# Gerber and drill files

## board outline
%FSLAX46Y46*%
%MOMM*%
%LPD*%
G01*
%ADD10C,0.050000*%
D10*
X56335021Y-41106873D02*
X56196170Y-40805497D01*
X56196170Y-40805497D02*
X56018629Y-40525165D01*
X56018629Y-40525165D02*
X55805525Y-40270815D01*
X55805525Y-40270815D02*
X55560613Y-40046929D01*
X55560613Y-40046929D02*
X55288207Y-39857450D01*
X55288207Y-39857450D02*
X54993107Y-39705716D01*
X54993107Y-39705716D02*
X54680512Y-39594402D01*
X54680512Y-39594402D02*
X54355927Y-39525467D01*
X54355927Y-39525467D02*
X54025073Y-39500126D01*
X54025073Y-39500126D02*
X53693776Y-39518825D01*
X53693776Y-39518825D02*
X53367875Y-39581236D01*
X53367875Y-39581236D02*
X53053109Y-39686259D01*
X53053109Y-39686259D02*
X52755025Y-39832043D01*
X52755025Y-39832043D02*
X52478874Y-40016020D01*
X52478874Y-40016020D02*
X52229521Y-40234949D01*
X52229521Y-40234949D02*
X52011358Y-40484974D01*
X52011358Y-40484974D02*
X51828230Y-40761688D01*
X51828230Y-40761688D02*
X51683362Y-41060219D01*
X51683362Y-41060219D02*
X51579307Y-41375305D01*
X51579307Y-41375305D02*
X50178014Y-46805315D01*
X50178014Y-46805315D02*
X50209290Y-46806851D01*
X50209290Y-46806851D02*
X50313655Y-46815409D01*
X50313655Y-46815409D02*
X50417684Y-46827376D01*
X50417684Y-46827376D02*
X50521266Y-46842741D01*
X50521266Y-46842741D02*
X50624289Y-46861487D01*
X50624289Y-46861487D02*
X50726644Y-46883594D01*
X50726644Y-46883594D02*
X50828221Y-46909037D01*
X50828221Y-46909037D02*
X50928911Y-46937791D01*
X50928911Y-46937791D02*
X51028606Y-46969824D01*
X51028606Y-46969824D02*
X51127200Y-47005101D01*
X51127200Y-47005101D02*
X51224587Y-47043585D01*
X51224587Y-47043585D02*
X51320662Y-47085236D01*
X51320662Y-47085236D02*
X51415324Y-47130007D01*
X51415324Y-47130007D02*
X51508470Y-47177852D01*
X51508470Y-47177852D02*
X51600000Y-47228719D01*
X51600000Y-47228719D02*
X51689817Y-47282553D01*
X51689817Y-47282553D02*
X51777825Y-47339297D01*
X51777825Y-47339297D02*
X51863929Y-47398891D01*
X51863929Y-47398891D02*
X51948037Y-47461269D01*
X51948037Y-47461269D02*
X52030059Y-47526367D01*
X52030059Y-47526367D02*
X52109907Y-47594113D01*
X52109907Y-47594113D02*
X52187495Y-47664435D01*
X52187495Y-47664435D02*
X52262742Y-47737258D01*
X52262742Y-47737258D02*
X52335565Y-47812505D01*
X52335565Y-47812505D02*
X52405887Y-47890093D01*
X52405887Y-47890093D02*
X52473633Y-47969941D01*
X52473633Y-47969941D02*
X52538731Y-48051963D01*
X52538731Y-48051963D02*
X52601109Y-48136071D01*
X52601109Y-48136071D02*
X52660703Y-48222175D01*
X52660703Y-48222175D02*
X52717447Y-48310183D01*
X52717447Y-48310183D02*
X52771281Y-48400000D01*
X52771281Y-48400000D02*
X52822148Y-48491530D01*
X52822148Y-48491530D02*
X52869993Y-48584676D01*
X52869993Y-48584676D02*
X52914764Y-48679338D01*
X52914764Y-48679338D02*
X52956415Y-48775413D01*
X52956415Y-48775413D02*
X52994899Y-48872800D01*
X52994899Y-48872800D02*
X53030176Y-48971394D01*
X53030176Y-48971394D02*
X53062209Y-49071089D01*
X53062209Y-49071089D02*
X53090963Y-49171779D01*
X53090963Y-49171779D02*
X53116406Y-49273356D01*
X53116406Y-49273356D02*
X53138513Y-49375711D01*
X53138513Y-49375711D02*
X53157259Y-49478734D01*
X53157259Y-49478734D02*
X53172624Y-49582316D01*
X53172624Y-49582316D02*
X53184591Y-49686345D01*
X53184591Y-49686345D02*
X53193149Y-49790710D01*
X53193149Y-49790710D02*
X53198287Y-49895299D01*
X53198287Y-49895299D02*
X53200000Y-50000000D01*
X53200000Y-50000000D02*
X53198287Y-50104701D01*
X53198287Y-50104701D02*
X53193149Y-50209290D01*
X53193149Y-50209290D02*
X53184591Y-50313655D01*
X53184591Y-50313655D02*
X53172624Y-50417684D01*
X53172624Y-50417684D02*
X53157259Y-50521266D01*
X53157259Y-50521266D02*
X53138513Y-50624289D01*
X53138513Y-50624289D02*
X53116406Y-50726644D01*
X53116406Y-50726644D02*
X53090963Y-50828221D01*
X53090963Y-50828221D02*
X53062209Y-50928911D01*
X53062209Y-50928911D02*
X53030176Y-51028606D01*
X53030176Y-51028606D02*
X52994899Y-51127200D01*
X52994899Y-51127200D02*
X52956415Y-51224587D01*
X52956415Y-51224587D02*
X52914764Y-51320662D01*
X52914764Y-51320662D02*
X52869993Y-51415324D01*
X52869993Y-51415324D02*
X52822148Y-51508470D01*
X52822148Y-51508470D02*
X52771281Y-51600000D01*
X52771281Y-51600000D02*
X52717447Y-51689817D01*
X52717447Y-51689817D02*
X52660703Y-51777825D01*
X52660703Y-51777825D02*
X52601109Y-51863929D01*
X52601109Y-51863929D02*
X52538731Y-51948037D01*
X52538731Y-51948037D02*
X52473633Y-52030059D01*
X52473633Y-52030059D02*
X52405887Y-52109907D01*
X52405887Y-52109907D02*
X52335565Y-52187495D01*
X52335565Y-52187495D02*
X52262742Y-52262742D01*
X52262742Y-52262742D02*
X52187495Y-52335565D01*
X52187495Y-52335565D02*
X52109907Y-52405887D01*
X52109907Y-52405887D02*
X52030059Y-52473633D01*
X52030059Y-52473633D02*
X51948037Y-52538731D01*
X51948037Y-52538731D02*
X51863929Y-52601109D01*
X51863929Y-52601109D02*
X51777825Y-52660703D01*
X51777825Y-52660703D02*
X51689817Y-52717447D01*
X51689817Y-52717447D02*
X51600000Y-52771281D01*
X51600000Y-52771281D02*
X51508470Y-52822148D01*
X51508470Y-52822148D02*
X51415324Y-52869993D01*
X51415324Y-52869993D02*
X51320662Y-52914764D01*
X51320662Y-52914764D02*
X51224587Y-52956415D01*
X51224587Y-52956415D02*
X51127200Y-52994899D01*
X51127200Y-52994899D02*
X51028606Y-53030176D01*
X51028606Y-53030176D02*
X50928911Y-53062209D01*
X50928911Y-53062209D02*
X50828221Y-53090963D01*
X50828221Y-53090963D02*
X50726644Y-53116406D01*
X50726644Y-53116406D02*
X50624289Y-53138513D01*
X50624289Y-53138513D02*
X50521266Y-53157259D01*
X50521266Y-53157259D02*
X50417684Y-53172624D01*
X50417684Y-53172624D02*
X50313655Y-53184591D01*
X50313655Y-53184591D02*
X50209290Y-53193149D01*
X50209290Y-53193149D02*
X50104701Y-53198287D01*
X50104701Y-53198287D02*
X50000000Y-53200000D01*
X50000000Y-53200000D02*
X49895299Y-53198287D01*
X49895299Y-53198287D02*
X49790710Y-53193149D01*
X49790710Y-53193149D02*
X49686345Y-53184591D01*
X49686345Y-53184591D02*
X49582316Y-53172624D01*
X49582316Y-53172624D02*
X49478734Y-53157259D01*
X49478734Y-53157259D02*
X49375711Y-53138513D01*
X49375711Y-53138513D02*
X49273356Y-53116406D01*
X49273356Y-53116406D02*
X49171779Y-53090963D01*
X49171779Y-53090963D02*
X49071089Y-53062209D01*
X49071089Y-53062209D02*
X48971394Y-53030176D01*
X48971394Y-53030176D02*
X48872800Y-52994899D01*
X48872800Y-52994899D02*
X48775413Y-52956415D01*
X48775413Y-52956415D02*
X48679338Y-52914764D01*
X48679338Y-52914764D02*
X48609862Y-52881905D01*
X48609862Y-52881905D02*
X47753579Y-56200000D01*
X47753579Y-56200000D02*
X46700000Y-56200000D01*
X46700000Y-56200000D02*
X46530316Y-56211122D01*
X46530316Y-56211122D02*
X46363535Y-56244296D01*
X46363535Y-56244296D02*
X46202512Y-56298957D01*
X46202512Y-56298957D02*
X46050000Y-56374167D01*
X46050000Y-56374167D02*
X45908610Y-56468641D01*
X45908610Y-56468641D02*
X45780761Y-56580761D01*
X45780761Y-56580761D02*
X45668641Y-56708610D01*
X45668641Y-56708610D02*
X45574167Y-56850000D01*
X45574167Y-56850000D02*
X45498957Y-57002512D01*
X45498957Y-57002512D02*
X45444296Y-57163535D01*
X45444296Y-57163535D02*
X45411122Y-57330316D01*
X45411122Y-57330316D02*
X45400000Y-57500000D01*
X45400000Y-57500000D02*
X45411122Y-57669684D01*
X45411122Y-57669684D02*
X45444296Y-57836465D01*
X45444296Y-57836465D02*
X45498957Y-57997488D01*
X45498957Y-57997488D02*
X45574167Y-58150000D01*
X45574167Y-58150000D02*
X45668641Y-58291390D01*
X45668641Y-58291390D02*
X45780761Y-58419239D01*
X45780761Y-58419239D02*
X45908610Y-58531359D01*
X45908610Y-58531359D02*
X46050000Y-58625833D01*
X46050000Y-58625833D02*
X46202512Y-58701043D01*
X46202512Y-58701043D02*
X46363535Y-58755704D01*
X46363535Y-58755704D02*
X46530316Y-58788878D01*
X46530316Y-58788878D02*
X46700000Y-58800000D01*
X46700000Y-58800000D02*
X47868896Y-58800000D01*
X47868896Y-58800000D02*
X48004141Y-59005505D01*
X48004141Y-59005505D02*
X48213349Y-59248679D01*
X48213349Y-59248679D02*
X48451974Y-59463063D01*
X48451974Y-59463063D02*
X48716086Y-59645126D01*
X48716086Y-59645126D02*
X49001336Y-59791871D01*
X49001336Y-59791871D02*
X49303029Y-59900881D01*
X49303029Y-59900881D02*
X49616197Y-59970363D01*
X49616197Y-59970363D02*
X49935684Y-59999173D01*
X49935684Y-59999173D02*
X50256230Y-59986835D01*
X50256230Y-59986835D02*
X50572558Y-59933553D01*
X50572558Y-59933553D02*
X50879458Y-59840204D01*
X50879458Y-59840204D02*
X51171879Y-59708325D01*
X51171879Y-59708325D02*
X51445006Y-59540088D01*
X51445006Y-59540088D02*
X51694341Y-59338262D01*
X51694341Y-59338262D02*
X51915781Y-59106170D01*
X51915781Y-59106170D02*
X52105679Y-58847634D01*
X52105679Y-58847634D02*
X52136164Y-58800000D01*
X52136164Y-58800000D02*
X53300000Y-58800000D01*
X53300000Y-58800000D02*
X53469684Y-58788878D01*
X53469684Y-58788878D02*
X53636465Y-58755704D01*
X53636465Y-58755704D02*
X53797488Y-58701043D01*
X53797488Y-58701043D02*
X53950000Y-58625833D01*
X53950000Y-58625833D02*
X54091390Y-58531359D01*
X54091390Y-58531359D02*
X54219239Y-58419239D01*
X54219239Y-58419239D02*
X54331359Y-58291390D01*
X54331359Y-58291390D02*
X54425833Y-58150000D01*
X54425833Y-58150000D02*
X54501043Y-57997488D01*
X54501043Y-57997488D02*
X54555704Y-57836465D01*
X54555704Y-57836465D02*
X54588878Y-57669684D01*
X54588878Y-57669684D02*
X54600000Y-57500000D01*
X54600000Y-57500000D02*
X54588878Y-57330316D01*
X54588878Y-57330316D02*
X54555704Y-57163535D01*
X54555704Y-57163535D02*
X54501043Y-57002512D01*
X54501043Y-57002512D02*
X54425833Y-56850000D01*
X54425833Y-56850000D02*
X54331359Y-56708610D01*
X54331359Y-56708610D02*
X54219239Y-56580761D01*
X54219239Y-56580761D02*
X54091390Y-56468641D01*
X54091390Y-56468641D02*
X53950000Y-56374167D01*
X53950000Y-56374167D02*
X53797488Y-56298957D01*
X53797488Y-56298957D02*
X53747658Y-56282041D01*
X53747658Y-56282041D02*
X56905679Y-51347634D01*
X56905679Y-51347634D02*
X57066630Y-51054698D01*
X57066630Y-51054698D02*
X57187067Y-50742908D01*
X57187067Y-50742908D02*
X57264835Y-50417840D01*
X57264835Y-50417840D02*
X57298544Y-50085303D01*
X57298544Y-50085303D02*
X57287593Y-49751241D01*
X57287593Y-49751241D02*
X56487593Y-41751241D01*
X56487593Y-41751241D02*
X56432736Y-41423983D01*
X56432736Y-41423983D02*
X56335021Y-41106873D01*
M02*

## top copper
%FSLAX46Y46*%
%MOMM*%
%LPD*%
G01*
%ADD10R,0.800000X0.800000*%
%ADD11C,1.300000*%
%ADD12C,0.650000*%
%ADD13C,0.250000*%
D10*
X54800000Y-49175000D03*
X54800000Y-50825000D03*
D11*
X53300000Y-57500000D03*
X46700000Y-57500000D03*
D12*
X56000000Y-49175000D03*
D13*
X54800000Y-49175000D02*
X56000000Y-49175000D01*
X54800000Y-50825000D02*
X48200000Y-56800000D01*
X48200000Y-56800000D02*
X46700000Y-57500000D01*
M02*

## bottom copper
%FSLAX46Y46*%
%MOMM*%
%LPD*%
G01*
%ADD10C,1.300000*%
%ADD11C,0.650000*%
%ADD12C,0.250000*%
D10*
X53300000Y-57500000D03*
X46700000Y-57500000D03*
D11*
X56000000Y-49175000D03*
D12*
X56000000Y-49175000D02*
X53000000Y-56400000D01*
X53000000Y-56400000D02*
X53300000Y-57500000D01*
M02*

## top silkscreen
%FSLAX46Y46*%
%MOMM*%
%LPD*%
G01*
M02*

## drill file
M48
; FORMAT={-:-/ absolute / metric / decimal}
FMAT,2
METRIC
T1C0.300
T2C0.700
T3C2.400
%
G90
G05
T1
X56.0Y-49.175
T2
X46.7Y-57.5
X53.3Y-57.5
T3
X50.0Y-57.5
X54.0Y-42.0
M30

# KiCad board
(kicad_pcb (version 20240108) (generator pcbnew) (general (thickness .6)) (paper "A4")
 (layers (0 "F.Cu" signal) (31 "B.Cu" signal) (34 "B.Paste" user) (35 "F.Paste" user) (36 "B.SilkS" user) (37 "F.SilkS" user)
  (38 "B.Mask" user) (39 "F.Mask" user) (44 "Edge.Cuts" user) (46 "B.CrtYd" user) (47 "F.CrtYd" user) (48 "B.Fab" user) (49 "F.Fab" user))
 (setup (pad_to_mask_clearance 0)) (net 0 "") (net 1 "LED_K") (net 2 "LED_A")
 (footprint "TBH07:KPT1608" (layer "F.Cu") (at 54.8 50)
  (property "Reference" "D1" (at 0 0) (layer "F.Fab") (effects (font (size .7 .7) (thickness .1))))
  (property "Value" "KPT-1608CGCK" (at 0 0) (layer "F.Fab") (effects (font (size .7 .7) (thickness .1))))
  (pad "1" smd rect (at 0 -.825) (size .8 .8) (layers "F.Cu" "F.Paste" "F.Mask") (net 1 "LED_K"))
  (pad "2" smd rect (at 0 .825) (size .8 .8) (layers "F.Cu" "F.Paste" "F.Mask") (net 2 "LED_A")))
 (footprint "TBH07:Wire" (layer "F.Cu") (at 53.3 57.5)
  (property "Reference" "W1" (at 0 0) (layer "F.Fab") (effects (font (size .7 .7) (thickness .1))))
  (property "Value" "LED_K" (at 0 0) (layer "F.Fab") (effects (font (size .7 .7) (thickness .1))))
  (pad "1" thru_hole circle (at 0 0) (size 1.3 1.3) (drill .7) (layers "*.Cu" "*.Mask") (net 1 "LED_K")))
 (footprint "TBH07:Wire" (layer "F.Cu") (at 46.7 57.5)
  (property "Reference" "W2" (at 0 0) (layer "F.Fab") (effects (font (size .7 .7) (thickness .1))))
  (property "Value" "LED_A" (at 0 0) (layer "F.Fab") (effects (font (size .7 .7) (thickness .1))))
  (pad "1" thru_hole circle (at 0 0) (size 1.3 1.3) (drill .7) (layers "*.Cu" "*.Mask") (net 2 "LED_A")))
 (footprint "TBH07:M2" (layer "F.Cu") (at 54 42)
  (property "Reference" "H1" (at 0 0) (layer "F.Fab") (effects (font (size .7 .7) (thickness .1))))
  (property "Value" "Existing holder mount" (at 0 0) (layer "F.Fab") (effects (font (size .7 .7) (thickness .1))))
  (pad "" np_thru_hole circle (at 0 0) (size 2.4 2.4) (drill 2.4) (layers "*.Cu" "*.Mask")))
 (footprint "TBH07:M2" (layer "F.Cu") (at 50 57.5)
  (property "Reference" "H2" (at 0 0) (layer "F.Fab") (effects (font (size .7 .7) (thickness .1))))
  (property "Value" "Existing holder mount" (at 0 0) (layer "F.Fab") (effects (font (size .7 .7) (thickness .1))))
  (pad "" np_thru_hole circle (at 0 0) (size 2.4 2.4) (drill 2.4) (layers "*.Cu" "*.Mask")))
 (segment (start 54.8 49.175) (end 56 49.175) (width .25) (layer "F.Cu") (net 1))
 (via (at 56 49.175) (size .65) (drill .3) (layers "F.Cu" "B.Cu") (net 1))
 (segment (start 56 49.175) (end 53.0 56.4) (width .25) (layer "B.Cu") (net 1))
 (segment (start 53.0 56.4) (end 53.3 57.5) (width .25) (layer "B.Cu") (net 1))
 (segment (start 54.8 50.825) (end 48.2 56.8) (width .25) (layer "F.Cu") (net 2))
 (segment (start 48.2 56.8) (end 46.7 57.5) (width .25) (layer "F.Cu") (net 2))
 (gr_line (start 56.33502112309573 41.106872710809505) (end 56.19616994221303 40.80549692971512) (stroke (width .05) (type default))
  (layer "Edge.Cuts"))
 (gr_line (start 56.19616994221303 40.80549692971512) (end 56.018628567749545 40.525164854817525) (stroke (width .05) (type default))
  (layer "Edge.Cuts"))
 (gr_line (start 56.018628567749545 40.525164854817525) (end 55.80552476774115 40.27081513045213) (stroke (width .05) (type default))
  (layer "Edge.Cuts"))
 (gr_line (start 55.80552476774115 40.27081513045213) (end 55.56061281780951 40.04692866671782) (stroke (width .05) (type default))
  (layer "Edge.Cuts"))
 (gr_line (start 55.56061281780951 40.04692866671782) (end 55.28820736163088 39.857449698737504) (stroke (width .05) (type default))
  (layer "Edge.Cuts"))
 (gr_line (start 55.28820736163088 39.857449698737504) (end 54.99310739933244 39.70571630058723) (stroke (width .05) (type default))
  (layer "Edge.Cuts"))
 (gr_line (start 54.99310739933244 39.70571630058723) (end 54.68051174292211 39.594401578038195) (stroke (width .05) (type default))
  (layer "Edge.Cuts"))
 (gr_line (start 54.68051174292211 39.594401578038195) (end 54.35592742818367 39.52546657612661) (stroke (width .05) (type default))
  (layer "Edge.Cuts"))
 (gr_line (start 54.35592742818367 39.52546657612661) (end 54.02507269655606 39.500125731184184) (stroke (width .05) (type default))
  (layer "Edge.Cuts"))
 (gr_line (start 54.02507269655606 39.500125731184184) (end 53.69377625617691 39.51882547596527) (stroke (width .05) (type default))
  (layer "Edge.Cuts"))
 (gr_line (start 53.69377625617691 39.51882547596527) (end 53.36787459682077 39.5812363747866) (stroke (width .05) (type default))
  (layer "Edge.Cuts"))
 (gr_line (start 53.36787459682077 39.5812363747866) (end 53.05310916774729 39.686258927235855) (stroke (width .05) (type default))
  (layer "Edge.Cuts"))
 (gr_line (start 53.05310916774729 39.686258927235855) (end 52.75502522988974 39.83204293820452) (stroke (width .05) (type default))
  (layer "Edge.Cuts"))
 (gr_line (start 52.75502522988974 39.83204293820452) (end 52.47887416431721 40.01602011300055) (stroke (width .05) (type default))
  (layer "Edge.Cuts"))
 (gr_line (start 52.47887416431721 40.01602011300055) (end 52.22952095801417 40.23494930330912) (stroke (width .05) (type default))
  (layer "Edge.Cuts"))
 (gr_line (start 52.22952095801417 40.23494930330912) (end 52.011358496811724 40.484973606897526) (stroke (width .05) (type default))
  (layer "Edge.Cuts"))
 (gr_line (start 52.011358496811724 40.484973606897526) (end 51.82823017538246 40.76168831513197) (stroke (width .05) (type default))
  (layer "Edge.Cuts"))
 (gr_line (start 51.82823017538246 40.76168831513197) (end 51.683362187687976 41.0602185112665) (stroke (width .05) (type default))
  (layer "Edge.Cuts"))
 (gr_line (start 51.683362187687976 41.0602185112665) (end 51.579306690726604 41.375304952445575) (stroke (width .05) (type default))
  (layer "Edge.Cuts"))
 (gr_line (start 51.579306690726604 41.375304952445575) (end 50.17801378986232 46.805314943294675) (stroke (width .05) (type default))
  (layer "Edge.Cuts"))
 (gr_line (start 50.17801378986232 46.805314943294675) (end 50.20929001353646 46.80685144563647) (stroke (width .05) (type default))
  (layer "Edge.Cuts"))
 (gr_line (start 50.20929001353646 46.80685144563647) (end 50.31365484905459 46.815408874648966) (stroke (width .05) (type default))
  (layer "Edge.Cuts"))
 (gr_line (start 50.31365484905459 46.815408874648966) (end 50.41768381510416 46.827376443603804) (stroke (width .05) (type default))
  (layer "Edge.Cuts"))
 (gr_line (start 50.41768381510416 46.827376443603804) (end 50.521265514862684 46.842741337328384) (stroke (width .05) (type default))
  (layer "Edge.Cuts"))
 (gr_line (start 50.521265514862684 46.842741337328384) (end 50.624289030451614 46.86148710270966) (stroke (width .05) (type default))
  (layer "Edge.Cuts"))
 (gr_line (start 50.624289030451614 46.86148710270966) (end 50.726644041709996 46.883593666312535) (stroke (width .05) (type default))
  (layer "Edge.Cuts"))
 (gr_line (start 50.726644041709996 46.883593666312535) (end 50.828220944328066 46.90903735587498) (stroke (width .05) (type default))
  (layer "Edge.Cuts"))
 (gr_line (start 50.828220944328066 46.90903735587498) (end 50.92891096721428 46.937790925656934) (stroke (width .05) (type default))
  (layer "Edge.Cuts"))
 (gr_line (start 50.92891096721428 46.937790925656934) (end 51.02860628897012 46.969823585615664) (stroke (width .05) (type default))
  (layer "Edge.Cuts"))
 (gr_line (start 51.02860628897012 46.969823585615664) (end 51.12720015334795 47.00510103437656) (stroke (width .05) (type default))
  (layer "Edge.Cuts"))
 (gr_line (start 51.12720015334795 47.00510103437656) (end 51.22458698356829 47.04358549596388) (stroke (width .05) (type default))
  (layer "Edge.Cuts"))
 (gr_line (start 51.22458698356829 47.04358549596388) (end 51.320662495374066 47.08523576025224) (stroke (width .05) (type default))
  (layer "Edge.Cuts"))
 (gr_line (start 51.320662495374066 47.08523576025224) (end 51.415323808700805 47.1300072270954) (stroke (width .05) (type default))
  (layer "Edge.Cuts"))
 (gr_line (start 51.415323808700805 47.1300072270954) (end 51.50846955784319 47.17785195408526) (stroke (width .05) (type default))
  (layer "Edge.Cuts"))
 (gr_line (start 51.50846955784319 47.17785195408526) (end 51.6 47.2287187078898) (stroke (width .05) (type default)) (layer "Edge.Cuts"))
 (gr_line (start 51.6 47.2287187078898) (end 51.68981712208118 47.28255301911495) (stroke (width .05) (type default)) (layer "Edge.Cuts"))
 (gr_line (start 51.68981712208118 47.28255301911495) (end 51.77782474566273 47.33929724063186) (stroke (width .05) (type default))
  (layer "Edge.Cuts"))
 (gr_line (start 51.77782474566273 47.33929724063186) (end 51.86392862997697 47.39889060930683) (stroke (width .05) (type default))
  (layer "Edge.Cuts"))
 (gr_line (start 51.86392862997697 47.39889060930683) (end 51.9480365728279 47.46126931106805) (stroke (width .05) (type default))
  (layer "Edge.Cuts"))
 (gr_line (start 51.9480365728279 47.46126931106805) (end 52.030058509323666 47.52636654923924) (stroke (width .05) (type default))
  (layer "Edge.Cuts"))
 (gr_line (start 52.030058509323666 47.52636654923924) (end 52.10990660832022 47.59411261606727) (stroke (width .05) (type default))
  (layer "Edge.Cuts"))
 (gr_line (start 52.10990660832022 47.59411261606727) (end 52.187495366473186 47.66443496736693) (stroke (width .05) (type default))
  (layer "Edge.Cuts"))
 (gr_line (start 52.187495366473186 47.66443496736693) (end 52.262741699796955 47.737258300203045) (stroke (width .05) (type default))
  (layer "Edge.Cuts"))
 (gr_line (start 52.262741699796955 47.737258300203045) (end 52.33556503263308 47.812504633526814) (stroke (width .05) (type default))
  (layer "Edge.Cuts"))
 (gr_line (start 52.33556503263308 47.812504633526814) (end 52.40588738393273 47.89009339167978) (stroke (width .05) (type default))
  (layer "Edge.Cuts"))
 (gr_line (start 52.40588738393273 47.89009339167978) (end 52.47363345076076 47.969941490676334) (stroke (width .05) (type default))
  (layer "Edge.Cuts"))
 (gr_line (start 52.47363345076076 47.969941490676334) (end 52.538730688931956 48.0519634271721) (stroke (width .05) (type default))
  (layer "Edge.Cuts"))
 (gr_line (start 52.538730688931956 48.0519634271721) (end 52.60110939069317 48.13607137002303) (stroke (width .05) (type default))
  (layer "Edge.Cuts"))
 (gr_line (start 52.60110939069317 48.13607137002303) (end 52.66070275936814 48.22217525433727) (stroke (width .05) (type default))
  (layer "Edge.Cuts"))
 (gr_line (start 52.66070275936814 48.22217525433727) (end 52.71744698088505 48.31018287791882) (stroke (width .05) (type default))
  (layer "Edge.Cuts"))
 (gr_line (start 52.71744698088505 48.31018287791882) (end 52.7712812921102 48.4) (stroke (width .05) (type default)) (layer "Edge.Cuts"))
 (gr_line (start 52.7712812921102 48.4) (end 52.82214804591474 48.49153044215681) (stroke (width .05) (type default)) (layer "Edge.Cuts"))
 (gr_line (start 52.82214804591474 48.49153044215681) (end 52.8699927729046 48.584676191299195) (stroke (width .05) (type default))
  (layer "Edge.Cuts"))
 (gr_line (start 52.8699927729046 48.584676191299195) (end 52.91476423974776 48.679337504625934) (stroke (width .05) (type default))
  (layer "Edge.Cuts"))
 (gr_line (start 52.91476423974776 48.679337504625934) (end 52.95641450403612 48.77541301643171) (stroke (width .05) (type default))
  (layer "Edge.Cuts"))
 (gr_line (start 52.95641450403612 48.77541301643171) (end 52.99489896562344 48.87279984665205) (stroke (width .05) (type default))
  (layer "Edge.Cuts"))
 (gr_line (start 52.99489896562344 48.87279984665205) (end 53.030176414384336 48.97139371102988) (stroke (width .05) (type default))
  (layer "Edge.Cuts"))
 (gr_line (start 53.030176414384336 48.97139371102988) (end 53.062209074343066 49.07108903278572) (stroke (width .05) (type default))
  (layer "Edge.Cuts"))
 (gr_line (start 53.062209074343066 49.07108903278572) (end 53.09096264412502 49.171779055671934) (stroke (width .05) (type default))
  (layer "Edge.Cuts"))
 (gr_line (start 53.09096264412502 49.171779055671934) (end 53.116406333687465 49.273355958290004) (stroke (width .05) (type default))
  (layer "Edge.Cuts"))
 (gr_line (start 53.116406333687465 49.273355958290004) (end 53.13851289729034 49.375710969548386) (stroke (width .05) (type default))
  (layer "Edge.Cuts"))
 (gr_line (start 53.13851289729034 49.375710969548386) (end 53.157258662671616 49.478734485137316) (stroke (width .05) (type default))
  (layer "Edge.Cuts"))
 (gr_line (start 53.157258662671616 49.478734485137316) (end 53.172623556396196 49.58231618489584) (stroke (width .05) (type default))
  (layer "Edge.Cuts"))
 (gr_line (start 53.172623556396196 49.58231618489584) (end 53.184591125351034 49.68634515094541) (stroke (width .05) (type default))
  (layer "Edge.Cuts"))
 (gr_line (start 53.184591125351034 49.68634515094541) (end 53.19314855436353 49.79070998646354) (stroke (width .05) (type default))
  (layer "Edge.Cuts"))
 (gr_line (start 53.19314855436353 49.79070998646354) (end 53.19828667992437 49.89529893497031) (stroke (width .05) (type default))
  (layer "Edge.Cuts"))
 (gr_line (start 53.19828667992437 49.89529893497031) (end 53.2 50.0) (stroke (width .05) (type default)) (layer "Edge.Cuts"))
 (gr_line (start 53.2 50.0) (end 53.19828667992437 50.10470106502969) (stroke (width .05) (type default)) (layer "Edge.Cuts"))
 (gr_line (start 53.19828667992437 50.10470106502969) (end 53.19314855436353 50.20929001353646) (stroke (width .05) (type default))
  (layer "Edge.Cuts"))
 (gr_line (start 53.19314855436353 50.20929001353646) (end 53.184591125351034 50.31365484905459) (stroke (width .05) (type default))
  (layer "Edge.Cuts"))
 (gr_line (start 53.184591125351034 50.31365484905459) (end 53.17262355639619 50.41768381510417) (stroke (width .05) (type default))
  (layer "Edge.Cuts"))
 (gr_line (start 53.17262355639619 50.41768381510417) (end 53.157258662671616 50.521265514862684) (stroke (width .05) (type default))
  (layer "Edge.Cuts"))
 (gr_line (start 53.157258662671616 50.521265514862684) (end 53.13851289729034 50.624289030451614) (stroke (width .05) (type default))
  (layer "Edge.Cuts"))
 (gr_line (start 53.13851289729034 50.624289030451614) (end 53.116406333687465 50.726644041709996) (stroke (width .05) (type default))
  (layer "Edge.Cuts"))
 (gr_line (start 53.116406333687465 50.726644041709996) (end 53.09096264412502 50.828220944328066) (stroke (width .05) (type default))
  (layer "Edge.Cuts"))
 (gr_line (start 53.09096264412502 50.828220944328066) (end 53.062209074343066 50.928910967214286) (stroke (width .05) (type default))
  (layer "Edge.Cuts"))
 (gr_line (start 53.062209074343066 50.928910967214286) (end 53.030176414384336 51.02860628897012) (stroke (width .05) (type default))
  (layer "Edge.Cuts"))
 (gr_line (start 53.030176414384336 51.02860628897012) (end 52.99489896562344 51.12720015334795) (stroke (width .05) (type default))
  (layer "Edge.Cuts"))
 (gr_line (start 52.99489896562344 51.12720015334795) (end 52.95641450403612 51.22458698356829) (stroke (width .05) (type default))
  (layer "Edge.Cuts"))
 (gr_line (start 52.95641450403612 51.22458698356829) (end 52.91476423974776 51.320662495374066) (stroke (width .05) (type default))
  (layer "Edge.Cuts"))
 (gr_line (start 52.91476423974776 51.320662495374066) (end 52.8699927729046 51.415323808700805) (stroke (width .05) (type default))
  (layer "Edge.Cuts"))
 (gr_line (start 52.8699927729046 51.415323808700805) (end 52.82214804591474 51.50846955784319) (stroke (width .05) (type default))
  (layer "Edge.Cuts"))
 (gr_line (start 52.82214804591474 51.50846955784319) (end 52.7712812921102 51.6) (stroke (width .05) (type default)) (layer "Edge.Cuts"))
 (gr_line (start 52.7712812921102 51.6) (end 52.71744698088505 51.68981712208118) (stroke (width .05) (type default)) (layer "Edge.Cuts"))
 (gr_line (start 52.71744698088505 51.68981712208118) (end 52.66070275936814 51.77782474566273) (stroke (width .05) (type default))
  (layer "Edge.Cuts"))
 (gr_line (start 52.66070275936814 51.77782474566273) (end 52.60110939069317 51.86392862997697) (stroke (width .05) (type default))
  (layer "Edge.Cuts"))
 (gr_line (start 52.60110939069317 51.86392862997697) (end 52.53873068893195 51.94803657282791) (stroke (width .05) (type default))
  (layer "Edge.Cuts"))
 (gr_line (start 52.53873068893195 51.94803657282791) (end 52.47363345076076 52.030058509323666) (stroke (width .05) (type default))
  (layer "Edge.Cuts"))
 (gr_line (start 52.47363345076076 52.030058509323666) (end 52.40588738393273 52.10990660832022) (stroke (width .05) (type default))
  (layer "Edge.Cuts"))
 (gr_line (start 52.40588738393273 52.10990660832022) (end 52.33556503263307 52.18749536647319) (stroke (width .05) (type default))
  (layer "Edge.Cuts"))
 (gr_line (start 52.33556503263307 52.18749536647319) (end 52.262741699796955 52.262741699796955) (stroke (width .05) (type default))
  (layer "Edge.Cuts"))
 (gr_line (start 52.262741699796955 52.262741699796955) (end 52.187495366473186 52.33556503263308) (stroke (width .05) (type default))
  (layer "Edge.Cuts"))
 (gr_line (start 52.187495366473186 52.33556503263308) (end 52.109906608320216 52.40588738393273) (stroke (width .05) (type default))
  (layer "Edge.Cuts"))
 (gr_line (start 52.109906608320216 52.40588738393273) (end 52.030058509323666 52.47363345076076) (stroke (width .05) (type default))
  (layer "Edge.Cuts"))
 (gr_line (start 52.030058509323666 52.47363345076076) (end 51.9480365728279 52.538730688931956) (stroke (width .05) (type default))
  (layer "Edge.Cuts"))
 (gr_line (start 51.9480365728279 52.538730688931956) (end 51.86392862997697 52.60110939069317) (stroke (width .05) (type default))
  (layer "Edge.Cuts"))
 (gr_line (start 51.86392862997697 52.60110939069317) (end 51.77782474566273 52.66070275936815) (stroke (width .05) (type default))
  (layer "Edge.Cuts"))
 (gr_line (start 51.77782474566273 52.66070275936815) (end 51.68981712208117 52.71744698088506) (stroke (width .05) (type default))
  (layer "Edge.Cuts"))
 (gr_line (start 51.68981712208117 52.71744698088506) (end 51.599999999999994 52.7712812921102) (stroke (width .05) (type default))
  (layer "Edge.Cuts"))
 (gr_line (start 51.599999999999994 52.7712812921102) (end 51.50846955784319 52.82214804591474) (stroke (width .05) (type default))
  (layer "Edge.Cuts"))
 (gr_line (start 51.50846955784319 52.82214804591474) (end 51.415323808700805 52.8699927729046) (stroke (width .05) (type default))
  (layer "Edge.Cuts"))
 (gr_line (start 51.415323808700805 52.8699927729046) (end 51.32066249537406 52.91476423974776) (stroke (width .05) (type default))
  (layer "Edge.Cuts"))
 (gr_line (start 51.32066249537406 52.91476423974776) (end 51.22458698356829 52.95641450403612) (stroke (width .05) (type default))
  (layer "Edge.Cuts"))
 (gr_line (start 51.22458698356829 52.95641450403612) (end 51.12720015334794 52.99489896562344) (stroke (width .05) (type default))
  (layer "Edge.Cuts"))
 (gr_line (start 51.12720015334794 52.99489896562344) (end 51.02860628897012 53.030176414384336) (stroke (width .05) (type default))
  (layer "Edge.Cuts"))
 (gr_line (start 51.02860628897012 53.030176414384336) (end 50.92891096721428 53.062209074343066) (stroke (width .05) (type default))
  (layer "Edge.Cuts"))
 (gr_line (start 50.92891096721428 53.062209074343066) (end 50.828220944328066 53.09096264412502) (stroke (width .05) (type default))
  (layer "Edge.Cuts"))
 (gr_line (start 50.828220944328066 53.09096264412502) (end 50.72664404170999 53.116406333687465) (stroke (width .05) (type default))
  (layer "Edge.Cuts"))
 (gr_line (start 50.72664404170999 53.116406333687465) (end 50.62428903045161 53.13851289729034) (stroke (width .05) (type default))
  (layer "Edge.Cuts"))
 (gr_line (start 50.62428903045161 53.13851289729034) (end 50.521265514862684 53.157258662671616) (stroke (width .05) (type default))
  (layer "Edge.Cuts"))
 (gr_line (start 50.521265514862684 53.157258662671616) (end 50.41768381510416 53.172623556396196) (stroke (width .05) (type default))
  (layer "Edge.Cuts"))
 (gr_line (start 50.41768381510416 53.172623556396196) (end 50.31365484905459 53.184591125351034) (stroke (width .05) (type default))
  (layer "Edge.Cuts"))
 (gr_line (start 50.31365484905459 53.184591125351034) (end 50.20929001353645 53.19314855436353) (stroke (width .05) (type default))
  (layer "Edge.Cuts"))
 (gr_line (start 50.20929001353645 53.19314855436353) (end 50.10470106502968 53.19828667992437) (stroke (width .05) (type default))
  (layer "Edge.Cuts"))
 (gr_line (start 50.10470106502968 53.19828667992437) (end 50.0 53.2) (stroke (width .05) (type default)) (layer "Edge.Cuts"))
 (gr_line (start 50.0 53.2) (end 49.89529893497031 53.19828667992437) (stroke (width .05) (type default)) (layer "Edge.Cuts"))
 (gr_line (start 49.89529893497031 53.19828667992437) (end 49.79070998646354 53.19314855436353) (stroke (width .05) (type default))
  (layer "Edge.Cuts"))
 (gr_line (start 49.79070998646354 53.19314855436353) (end 49.68634515094541 53.184591125351034) (stroke (width .05) (type default))
  (layer "Edge.Cuts"))
 (gr_line (start 49.68634515094541 53.184591125351034) (end 49.58231618489583 53.17262355639619) (stroke (width .05) (type default))
  (layer "Edge.Cuts"))
 (gr_line (start 49.58231618489583 53.17262355639619) (end 49.478734485137316 53.157258662671616) (stroke (width .05) (type default))
  (layer "Edge.Cuts"))
 (gr_line (start 49.478734485137316 53.157258662671616) (end 49.375710969548386 53.13851289729034) (stroke (width .05) (type default))
  (layer "Edge.Cuts"))
 (gr_line (start 49.375710969548386 53.13851289729034) (end 49.273355958290004 53.116406333687465) (stroke (width .05) (type default))
  (layer "Edge.Cuts"))
 (gr_line (start 49.273355958290004 53.116406333687465) (end 49.171779055671934 53.09096264412502) (stroke (width .05) (type default))
  (layer "Edge.Cuts"))
 (gr_line (start 49.171779055671934 53.09096264412502) (end 49.07108903278572 53.062209074343066) (stroke (width .05) (type default))
  (layer "Edge.Cuts"))
 (gr_line (start 49.07108903278572 53.062209074343066) (end 48.97139371102988 53.030176414384336) (stroke (width .05) (type default))
  (layer "Edge.Cuts"))
 (gr_line (start 48.97139371102988 53.030176414384336) (end 48.87279984665205 52.99489896562344) (stroke (width .05) (type default))
  (layer "Edge.Cuts"))
 (gr_line (start 48.87279984665205 52.99489896562344) (end 48.77541301643171 52.95641450403612) (stroke (width .05) (type default))
  (layer "Edge.Cuts"))
 (gr_line (start 48.77541301643171 52.95641450403612) (end 48.679337504625934 52.91476423974776) (stroke (width .05) (type default))
  (layer "Edge.Cuts"))
 (gr_line (start 48.679337504625934 52.91476423974776) (end 48.609861621831975 52.88190459441226) (stroke (width .05) (type default))
  (layer "Edge.Cuts"))
 (gr_line (start 48.609861621831975 52.88190459441226) (end 47.75357893651901 56.2) (stroke (width .05) (type default)) (layer "Edge.Cuts"))
 (gr_line (start 47.75357893651901 56.2) (end 46.7 56.2) (stroke (width .05) (type default)) (layer "Edge.Cuts"))
 (gr_line (start 46.7 56.2) (end 46.53031595011393 56.21112168021405) (stroke (width .05) (type default)) (layer "Edge.Cuts"))
 (gr_line (start 46.53031595011393 56.21112168021405) (end 46.363535241366726 56.24429642582421) (stroke (width .05) (type default))
  (layer "Edge.Cuts"))
 (gr_line (start 46.363535241366726 56.24429642582421) (end 46.20251153792538 56.29895660773533) (stroke (width .05) (type default))
  (layer "Edge.Cuts"))
 (gr_line (start 46.20251153792538 56.29895660773533) (end 46.05 56.37416697508023) (stroke (width .05) (type default)) (layer "Edge.Cuts"))
 (gr_line (start 46.05 56.37416697508023) (end 45.908610142288666 56.46864065762139) (stroke (width .05) (type default)) (layer "Edge.Cuts"))
 (gr_line (start 45.908610142288666 56.46864065762139) (end 45.78076118445749 56.58076118445749) (stroke (width .05) (type default))
  (layer "Edge.Cuts"))
 (gr_line (start 45.78076118445749 56.58076118445749) (end 45.668640657621395 56.70861014228866) (stroke (width .05) (type default))
  (layer "Edge.Cuts"))
 (gr_line (start 45.668640657621395 56.70861014228866) (end 45.57416697508023 56.85) (stroke (width .05) (type default)) (layer "Edge.Cuts"))
 (gr_line (start 45.57416697508023 56.85) (end 45.49895660773532 57.002511537925386) (stroke (width .05) (type default)) (layer "Edge.Cuts"))
 (gr_line (start 45.49895660773532 57.002511537925386) (end 45.44429642582421 57.16353524136672) (stroke (width .05) (type default))
  (layer "Edge.Cuts"))
 (gr_line (start 45.44429642582421 57.16353524136672) (end 45.411121680214045 57.330315950113935) (stroke (width .05) (type default))
  (layer "Edge.Cuts"))
 (gr_line (start 45.411121680214045 57.330315950113935) (end 45.4 57.5) (stroke (width .05) (type default)) (layer "Edge.Cuts"))
 (gr_line (start 45.4 57.5) (end 45.411121680214045 57.669684049886065) (stroke (width .05) (type default)) (layer "Edge.Cuts"))
 (gr_line (start 45.411121680214045 57.669684049886065) (end 45.44429642582421 57.83646475863328) (stroke (width .05) (type default))
  (layer "Edge.Cuts"))
 (gr_line (start 45.44429642582421 57.83646475863328) (end 45.49895660773532 57.997488462074614) (stroke (width .05) (type default))
  (layer "Edge.Cuts"))
 (gr_line (start 45.49895660773532 57.997488462074614) (end 45.57416697508023 58.15) (stroke (width .05) (type default)) (layer "Edge.Cuts"))
 (gr_line (start 45.57416697508023 58.15) (end 45.668640657621395 58.29138985771134) (stroke (width .05) (type default)) (layer "Edge.Cuts"))
 (gr_line (start 45.668640657621395 58.29138985771134) (end 45.78076118445749 58.41923881554251) (stroke (width .05) (type default))
  (layer "Edge.Cuts"))
 (gr_line (start 45.78076118445749 58.41923881554251) (end 45.908610142288666 58.53135934237861) (stroke (width .05) (type default))
  (layer "Edge.Cuts"))
 (gr_line (start 45.908610142288666 58.53135934237861) (end 46.05 58.62583302491977) (stroke (width .05) (type default)) (layer "Edge.Cuts"))
 (gr_line (start 46.05 58.62583302491977) (end 46.20251153792538 58.70104339226467) (stroke (width .05) (type default)) (layer "Edge.Cuts"))
 (gr_line (start 46.20251153792538 58.70104339226467) (end 46.363535241366726 58.75570357417579) (stroke (width .05) (type default))
  (layer "Edge.Cuts"))
 (gr_line (start 46.363535241366726 58.75570357417579) (end 46.53031595011393 58.78887831978595) (stroke (width .05) (type default))
  (layer "Edge.Cuts"))
 (gr_line (start 46.53031595011393 58.78887831978595) (end 46.7 58.8) (stroke (width .05) (type default)) (layer "Edge.Cuts"))
 (gr_line (start 46.7 58.8) (end 47.86889561311338 58.8) (stroke (width .05) (type default)) (layer "Edge.Cuts"))
 (gr_line (start 47.86889561311338 58.8) (end 48.004140612218805 59.00550499972789) (stroke (width .05) (type default)) (layer "Edge.Cuts"))
 (gr_line (start 48.004140612218805 59.00550499972789) (end 48.213349249283795 59.24867924301892) (stroke (width .05) (type default))
  (layer "Edge.Cuts"))
 (gr_line (start 48.213349249283795 59.24867924301892) (end 48.45197386643828 59.463062681070056) (stroke (width .05) (type default))
  (layer "Edge.Cuts"))
 (gr_line (start 48.45197386643828 59.463062681070056) (end 48.71608567290754 59.64512563750628) (stroke (width .05) (type default))
  (layer "Edge.Cuts"))
 (gr_line (start 48.71608567290754 59.64512563750628) (end 49.00133624881299 59.791870570530776) (stroke (width .05) (type default))
  (layer "Edge.Cuts"))
 (gr_line (start 49.00133624881299 59.791870570530776) (end 49.3030291389252 59.900881425396236) (stroke (width .05) (type default))
  (layer "Edge.Cuts"))
 (gr_line (start 49.3030291389252 59.900881425396236) (end 49.616197176580435 59.970363413090304) (stroke (width .05) (type default))
  (layer "Edge.Cuts"))
 (gr_line (start 49.616197176580435 59.970363413090304) (end 49.93568426467543 59.99917256030665) (stroke (width .05) (type default))
  (layer "Edge.Cuts"))
 (gr_line (start 49.93568426467543 59.99917256030665) (end 50.25623026727232 59.98683454418133) (stroke (width .05) (type default))
  (layer "Edge.Cuts"))
 (gr_line (start 50.25623026727232 59.98683454418133) (end 50.57255761413172 59.933552501693725) (stroke (width .05) (type default))
  (layer "Edge.Cuts"))
 (gr_line (start 50.57255761413172 59.933552501693725) (end 50.87945819228959 59.84020368515536) (stroke (width .05) (type default))
  (layer "Edge.Cuts"))
 (gr_line (start 50.87945819228959 59.84020368515536) (end 51.171879094067755 59.70832501885183) (stroke (width .05) (type default))
  (layer "Edge.Cuts"))
 (gr_line (start 51.171879094067755 59.70832501885183) (end 51.44500580973563 59.540087794637834) (stroke (width .05) (type default))
  (layer "Edge.Cuts"))
 (gr_line (start 51.44500580973563 59.540087794637834) (end 51.694341495113264 59.33826192310491) (stroke (width .05) (type default))
  (layer "Edge.Cuts"))
 (gr_line (start 51.694341495113264 59.33826192310491) (end 51.91578100902867 59.106170328901975) (stroke (width .05) (type default))
  (layer "Edge.Cuts"))
 (gr_line (start 51.91578100902867 59.106170328901975) (end 52.10567850165378 58.847634241058415) (stroke (width .05) (type default))
  (layer "Edge.Cuts"))
 (gr_line (start 52.10567850165378 58.847634241058415) (end 52.13616441593116 58.8) (stroke (width .05) (type default)) (layer "Edge.Cuts"))
 (gr_line (start 52.13616441593116 58.8) (end 53.3 58.8) (stroke (width .05) (type default)) (layer "Edge.Cuts"))
 (gr_line (start 53.3 58.8) (end 53.46968404988607 58.78887831978595) (stroke (width .05) (type default)) (layer "Edge.Cuts"))
 (gr_line (start 53.46968404988607 58.78887831978595) (end 53.636464758633274 58.75570357417579) (stroke (width .05) (type default))
  (layer "Edge.Cuts"))
 (gr_line (start 53.636464758633274 58.75570357417579) (end 53.79748846207462 58.70104339226467) (stroke (width .05) (type default))
  (layer "Edge.Cuts"))
 (gr_line (start 53.79748846207462 58.70104339226467) (end 53.95 58.62583302491977) (stroke (width .05) (type default)) (layer "Edge.Cuts"))
 (gr_line (start 53.95 58.62583302491977) (end 54.091389857711334 58.53135934237861) (stroke (width .05) (type default)) (layer "Edge.Cuts"))
 (gr_line (start 54.091389857711334 58.53135934237861) (end 54.21923881554251 58.41923881554251) (stroke (width .05) (type default))
  (layer "Edge.Cuts"))
 (gr_line (start 54.21923881554251 58.41923881554251) (end 54.331359342378605 58.29138985771134) (stroke (width .05) (type default))
  (layer "Edge.Cuts"))
 (gr_line (start 54.331359342378605 58.29138985771134) (end 54.42583302491977 58.15) (stroke (width .05) (type default)) (layer "Edge.Cuts"))
 (gr_line (start 54.42583302491977 58.15) (end 54.50104339226467 57.997488462074614) (stroke (width .05) (type default)) (layer "Edge.Cuts"))
 (gr_line (start 54.50104339226467 57.997488462074614) (end 54.55570357417579 57.83646475863328) (stroke (width .05) (type default))
  (layer "Edge.Cuts"))
 (gr_line (start 54.55570357417579 57.83646475863328) (end 54.588878319785955 57.669684049886065) (stroke (width .05) (type default))
  (layer "Edge.Cuts"))
 (gr_line (start 54.588878319785955 57.669684049886065) (end 54.6 57.5) (stroke (width .05) (type default)) (layer "Edge.Cuts"))
 (gr_line (start 54.6 57.5) (end 54.588878319785955 57.330315950113935) (stroke (width .05) (type default)) (layer "Edge.Cuts"))
 (gr_line (start 54.588878319785955 57.330315950113935) (end 54.55570357417579 57.16353524136672) (stroke (width .05) (type default))
  (layer "Edge.Cuts"))
 (gr_line (start 54.55570357417579 57.16353524136672) (end 54.50104339226468 57.002511537925386) (stroke (width .05) (type default))
  (layer "Edge.Cuts"))
 (gr_line (start 54.50104339226468 57.002511537925386) (end 54.42583302491977 56.85) (stroke (width .05) (type default)) (layer "Edge.Cuts"))
 (gr_line (start 54.42583302491977 56.85) (end 54.331359342378605 56.70861014228866) (stroke (width .05) (type default)) (layer "Edge.Cuts"))
 (gr_line (start 54.331359342378605 56.70861014228866) (end 54.21923881554251 56.58076118445749) (stroke (width .05) (type default))
  (layer "Edge.Cuts"))
 (gr_line (start 54.21923881554251 56.58076118445749) (end 54.091389857711334 56.46864065762139) (stroke (width .05) (type default))
  (layer "Edge.Cuts"))
 (gr_line (start 54.091389857711334 56.46864065762139) (end 53.95 56.37416697508023) (stroke (width .05) (type default)) (layer "Edge.Cuts"))
 (gr_line (start 53.95 56.37416697508023) (end 53.79748846207462 56.29895660773533) (stroke (width .05) (type default)) (layer "Edge.Cuts"))
 (gr_line (start 53.79748846207462 56.29895660773533) (end 53.747657910476015 56.28204141477367) (stroke (width .05) (type default))
  (layer "Edge.Cuts"))
 (gr_line (start 53.747657910476015 56.28204141477367) (end 56.90567850165378 51.347634241058415) (stroke (width .05) (type default))
  (layer "Edge.Cuts"))
 (gr_line (start 56.90567850165378 51.347634241058415) (end 57.066630317166364 51.05469758950247) (stroke (width .05) (type default))
  (layer "Edge.Cuts"))
 (gr_line (start 57.066630317166364 51.05469758950247) (end 57.18706661668794 50.74290845162375) (stroke (width .05) (type default))
  (layer "Edge.Cuts"))
 (gr_line (start 57.18706661668794 50.74290845162375) (end 57.264834627981145 50.41783998935602) (stroke (width .05) (type default))
  (layer "Edge.Cuts"))
 (gr_line (start 57.264834627981145 50.41783998935602) (end 57.298544265030955 50.085302729621745) (stroke (width .05) (type default))
  (layer "Edge.Cuts"))
 (gr_line (start 57.298544265030955 50.085302729621745) (end 57.28759297552497 49.751240702447504) (stroke (width .05) (type default))
  (layer "Edge.Cuts"))
 (gr_line (start 57.28759297552497 49.751240702447504) (end 56.487592975524976 41.751240702447504) (stroke (width .05) (type default))
  (layer "Edge.Cuts"))
 (gr_line (start 56.487592975524976 41.751240702447504) (end 56.432735952218344 41.423982824228034) (stroke (width .05) (type default))
  (layer "Edge.Cuts"))
 (gr_line (start 56.432735952218344 41.423982824228034) (end 56.33502112309573 41.106872710809505) (stroke (width .05) (type default))
  (layer "Edge.Cuts")))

